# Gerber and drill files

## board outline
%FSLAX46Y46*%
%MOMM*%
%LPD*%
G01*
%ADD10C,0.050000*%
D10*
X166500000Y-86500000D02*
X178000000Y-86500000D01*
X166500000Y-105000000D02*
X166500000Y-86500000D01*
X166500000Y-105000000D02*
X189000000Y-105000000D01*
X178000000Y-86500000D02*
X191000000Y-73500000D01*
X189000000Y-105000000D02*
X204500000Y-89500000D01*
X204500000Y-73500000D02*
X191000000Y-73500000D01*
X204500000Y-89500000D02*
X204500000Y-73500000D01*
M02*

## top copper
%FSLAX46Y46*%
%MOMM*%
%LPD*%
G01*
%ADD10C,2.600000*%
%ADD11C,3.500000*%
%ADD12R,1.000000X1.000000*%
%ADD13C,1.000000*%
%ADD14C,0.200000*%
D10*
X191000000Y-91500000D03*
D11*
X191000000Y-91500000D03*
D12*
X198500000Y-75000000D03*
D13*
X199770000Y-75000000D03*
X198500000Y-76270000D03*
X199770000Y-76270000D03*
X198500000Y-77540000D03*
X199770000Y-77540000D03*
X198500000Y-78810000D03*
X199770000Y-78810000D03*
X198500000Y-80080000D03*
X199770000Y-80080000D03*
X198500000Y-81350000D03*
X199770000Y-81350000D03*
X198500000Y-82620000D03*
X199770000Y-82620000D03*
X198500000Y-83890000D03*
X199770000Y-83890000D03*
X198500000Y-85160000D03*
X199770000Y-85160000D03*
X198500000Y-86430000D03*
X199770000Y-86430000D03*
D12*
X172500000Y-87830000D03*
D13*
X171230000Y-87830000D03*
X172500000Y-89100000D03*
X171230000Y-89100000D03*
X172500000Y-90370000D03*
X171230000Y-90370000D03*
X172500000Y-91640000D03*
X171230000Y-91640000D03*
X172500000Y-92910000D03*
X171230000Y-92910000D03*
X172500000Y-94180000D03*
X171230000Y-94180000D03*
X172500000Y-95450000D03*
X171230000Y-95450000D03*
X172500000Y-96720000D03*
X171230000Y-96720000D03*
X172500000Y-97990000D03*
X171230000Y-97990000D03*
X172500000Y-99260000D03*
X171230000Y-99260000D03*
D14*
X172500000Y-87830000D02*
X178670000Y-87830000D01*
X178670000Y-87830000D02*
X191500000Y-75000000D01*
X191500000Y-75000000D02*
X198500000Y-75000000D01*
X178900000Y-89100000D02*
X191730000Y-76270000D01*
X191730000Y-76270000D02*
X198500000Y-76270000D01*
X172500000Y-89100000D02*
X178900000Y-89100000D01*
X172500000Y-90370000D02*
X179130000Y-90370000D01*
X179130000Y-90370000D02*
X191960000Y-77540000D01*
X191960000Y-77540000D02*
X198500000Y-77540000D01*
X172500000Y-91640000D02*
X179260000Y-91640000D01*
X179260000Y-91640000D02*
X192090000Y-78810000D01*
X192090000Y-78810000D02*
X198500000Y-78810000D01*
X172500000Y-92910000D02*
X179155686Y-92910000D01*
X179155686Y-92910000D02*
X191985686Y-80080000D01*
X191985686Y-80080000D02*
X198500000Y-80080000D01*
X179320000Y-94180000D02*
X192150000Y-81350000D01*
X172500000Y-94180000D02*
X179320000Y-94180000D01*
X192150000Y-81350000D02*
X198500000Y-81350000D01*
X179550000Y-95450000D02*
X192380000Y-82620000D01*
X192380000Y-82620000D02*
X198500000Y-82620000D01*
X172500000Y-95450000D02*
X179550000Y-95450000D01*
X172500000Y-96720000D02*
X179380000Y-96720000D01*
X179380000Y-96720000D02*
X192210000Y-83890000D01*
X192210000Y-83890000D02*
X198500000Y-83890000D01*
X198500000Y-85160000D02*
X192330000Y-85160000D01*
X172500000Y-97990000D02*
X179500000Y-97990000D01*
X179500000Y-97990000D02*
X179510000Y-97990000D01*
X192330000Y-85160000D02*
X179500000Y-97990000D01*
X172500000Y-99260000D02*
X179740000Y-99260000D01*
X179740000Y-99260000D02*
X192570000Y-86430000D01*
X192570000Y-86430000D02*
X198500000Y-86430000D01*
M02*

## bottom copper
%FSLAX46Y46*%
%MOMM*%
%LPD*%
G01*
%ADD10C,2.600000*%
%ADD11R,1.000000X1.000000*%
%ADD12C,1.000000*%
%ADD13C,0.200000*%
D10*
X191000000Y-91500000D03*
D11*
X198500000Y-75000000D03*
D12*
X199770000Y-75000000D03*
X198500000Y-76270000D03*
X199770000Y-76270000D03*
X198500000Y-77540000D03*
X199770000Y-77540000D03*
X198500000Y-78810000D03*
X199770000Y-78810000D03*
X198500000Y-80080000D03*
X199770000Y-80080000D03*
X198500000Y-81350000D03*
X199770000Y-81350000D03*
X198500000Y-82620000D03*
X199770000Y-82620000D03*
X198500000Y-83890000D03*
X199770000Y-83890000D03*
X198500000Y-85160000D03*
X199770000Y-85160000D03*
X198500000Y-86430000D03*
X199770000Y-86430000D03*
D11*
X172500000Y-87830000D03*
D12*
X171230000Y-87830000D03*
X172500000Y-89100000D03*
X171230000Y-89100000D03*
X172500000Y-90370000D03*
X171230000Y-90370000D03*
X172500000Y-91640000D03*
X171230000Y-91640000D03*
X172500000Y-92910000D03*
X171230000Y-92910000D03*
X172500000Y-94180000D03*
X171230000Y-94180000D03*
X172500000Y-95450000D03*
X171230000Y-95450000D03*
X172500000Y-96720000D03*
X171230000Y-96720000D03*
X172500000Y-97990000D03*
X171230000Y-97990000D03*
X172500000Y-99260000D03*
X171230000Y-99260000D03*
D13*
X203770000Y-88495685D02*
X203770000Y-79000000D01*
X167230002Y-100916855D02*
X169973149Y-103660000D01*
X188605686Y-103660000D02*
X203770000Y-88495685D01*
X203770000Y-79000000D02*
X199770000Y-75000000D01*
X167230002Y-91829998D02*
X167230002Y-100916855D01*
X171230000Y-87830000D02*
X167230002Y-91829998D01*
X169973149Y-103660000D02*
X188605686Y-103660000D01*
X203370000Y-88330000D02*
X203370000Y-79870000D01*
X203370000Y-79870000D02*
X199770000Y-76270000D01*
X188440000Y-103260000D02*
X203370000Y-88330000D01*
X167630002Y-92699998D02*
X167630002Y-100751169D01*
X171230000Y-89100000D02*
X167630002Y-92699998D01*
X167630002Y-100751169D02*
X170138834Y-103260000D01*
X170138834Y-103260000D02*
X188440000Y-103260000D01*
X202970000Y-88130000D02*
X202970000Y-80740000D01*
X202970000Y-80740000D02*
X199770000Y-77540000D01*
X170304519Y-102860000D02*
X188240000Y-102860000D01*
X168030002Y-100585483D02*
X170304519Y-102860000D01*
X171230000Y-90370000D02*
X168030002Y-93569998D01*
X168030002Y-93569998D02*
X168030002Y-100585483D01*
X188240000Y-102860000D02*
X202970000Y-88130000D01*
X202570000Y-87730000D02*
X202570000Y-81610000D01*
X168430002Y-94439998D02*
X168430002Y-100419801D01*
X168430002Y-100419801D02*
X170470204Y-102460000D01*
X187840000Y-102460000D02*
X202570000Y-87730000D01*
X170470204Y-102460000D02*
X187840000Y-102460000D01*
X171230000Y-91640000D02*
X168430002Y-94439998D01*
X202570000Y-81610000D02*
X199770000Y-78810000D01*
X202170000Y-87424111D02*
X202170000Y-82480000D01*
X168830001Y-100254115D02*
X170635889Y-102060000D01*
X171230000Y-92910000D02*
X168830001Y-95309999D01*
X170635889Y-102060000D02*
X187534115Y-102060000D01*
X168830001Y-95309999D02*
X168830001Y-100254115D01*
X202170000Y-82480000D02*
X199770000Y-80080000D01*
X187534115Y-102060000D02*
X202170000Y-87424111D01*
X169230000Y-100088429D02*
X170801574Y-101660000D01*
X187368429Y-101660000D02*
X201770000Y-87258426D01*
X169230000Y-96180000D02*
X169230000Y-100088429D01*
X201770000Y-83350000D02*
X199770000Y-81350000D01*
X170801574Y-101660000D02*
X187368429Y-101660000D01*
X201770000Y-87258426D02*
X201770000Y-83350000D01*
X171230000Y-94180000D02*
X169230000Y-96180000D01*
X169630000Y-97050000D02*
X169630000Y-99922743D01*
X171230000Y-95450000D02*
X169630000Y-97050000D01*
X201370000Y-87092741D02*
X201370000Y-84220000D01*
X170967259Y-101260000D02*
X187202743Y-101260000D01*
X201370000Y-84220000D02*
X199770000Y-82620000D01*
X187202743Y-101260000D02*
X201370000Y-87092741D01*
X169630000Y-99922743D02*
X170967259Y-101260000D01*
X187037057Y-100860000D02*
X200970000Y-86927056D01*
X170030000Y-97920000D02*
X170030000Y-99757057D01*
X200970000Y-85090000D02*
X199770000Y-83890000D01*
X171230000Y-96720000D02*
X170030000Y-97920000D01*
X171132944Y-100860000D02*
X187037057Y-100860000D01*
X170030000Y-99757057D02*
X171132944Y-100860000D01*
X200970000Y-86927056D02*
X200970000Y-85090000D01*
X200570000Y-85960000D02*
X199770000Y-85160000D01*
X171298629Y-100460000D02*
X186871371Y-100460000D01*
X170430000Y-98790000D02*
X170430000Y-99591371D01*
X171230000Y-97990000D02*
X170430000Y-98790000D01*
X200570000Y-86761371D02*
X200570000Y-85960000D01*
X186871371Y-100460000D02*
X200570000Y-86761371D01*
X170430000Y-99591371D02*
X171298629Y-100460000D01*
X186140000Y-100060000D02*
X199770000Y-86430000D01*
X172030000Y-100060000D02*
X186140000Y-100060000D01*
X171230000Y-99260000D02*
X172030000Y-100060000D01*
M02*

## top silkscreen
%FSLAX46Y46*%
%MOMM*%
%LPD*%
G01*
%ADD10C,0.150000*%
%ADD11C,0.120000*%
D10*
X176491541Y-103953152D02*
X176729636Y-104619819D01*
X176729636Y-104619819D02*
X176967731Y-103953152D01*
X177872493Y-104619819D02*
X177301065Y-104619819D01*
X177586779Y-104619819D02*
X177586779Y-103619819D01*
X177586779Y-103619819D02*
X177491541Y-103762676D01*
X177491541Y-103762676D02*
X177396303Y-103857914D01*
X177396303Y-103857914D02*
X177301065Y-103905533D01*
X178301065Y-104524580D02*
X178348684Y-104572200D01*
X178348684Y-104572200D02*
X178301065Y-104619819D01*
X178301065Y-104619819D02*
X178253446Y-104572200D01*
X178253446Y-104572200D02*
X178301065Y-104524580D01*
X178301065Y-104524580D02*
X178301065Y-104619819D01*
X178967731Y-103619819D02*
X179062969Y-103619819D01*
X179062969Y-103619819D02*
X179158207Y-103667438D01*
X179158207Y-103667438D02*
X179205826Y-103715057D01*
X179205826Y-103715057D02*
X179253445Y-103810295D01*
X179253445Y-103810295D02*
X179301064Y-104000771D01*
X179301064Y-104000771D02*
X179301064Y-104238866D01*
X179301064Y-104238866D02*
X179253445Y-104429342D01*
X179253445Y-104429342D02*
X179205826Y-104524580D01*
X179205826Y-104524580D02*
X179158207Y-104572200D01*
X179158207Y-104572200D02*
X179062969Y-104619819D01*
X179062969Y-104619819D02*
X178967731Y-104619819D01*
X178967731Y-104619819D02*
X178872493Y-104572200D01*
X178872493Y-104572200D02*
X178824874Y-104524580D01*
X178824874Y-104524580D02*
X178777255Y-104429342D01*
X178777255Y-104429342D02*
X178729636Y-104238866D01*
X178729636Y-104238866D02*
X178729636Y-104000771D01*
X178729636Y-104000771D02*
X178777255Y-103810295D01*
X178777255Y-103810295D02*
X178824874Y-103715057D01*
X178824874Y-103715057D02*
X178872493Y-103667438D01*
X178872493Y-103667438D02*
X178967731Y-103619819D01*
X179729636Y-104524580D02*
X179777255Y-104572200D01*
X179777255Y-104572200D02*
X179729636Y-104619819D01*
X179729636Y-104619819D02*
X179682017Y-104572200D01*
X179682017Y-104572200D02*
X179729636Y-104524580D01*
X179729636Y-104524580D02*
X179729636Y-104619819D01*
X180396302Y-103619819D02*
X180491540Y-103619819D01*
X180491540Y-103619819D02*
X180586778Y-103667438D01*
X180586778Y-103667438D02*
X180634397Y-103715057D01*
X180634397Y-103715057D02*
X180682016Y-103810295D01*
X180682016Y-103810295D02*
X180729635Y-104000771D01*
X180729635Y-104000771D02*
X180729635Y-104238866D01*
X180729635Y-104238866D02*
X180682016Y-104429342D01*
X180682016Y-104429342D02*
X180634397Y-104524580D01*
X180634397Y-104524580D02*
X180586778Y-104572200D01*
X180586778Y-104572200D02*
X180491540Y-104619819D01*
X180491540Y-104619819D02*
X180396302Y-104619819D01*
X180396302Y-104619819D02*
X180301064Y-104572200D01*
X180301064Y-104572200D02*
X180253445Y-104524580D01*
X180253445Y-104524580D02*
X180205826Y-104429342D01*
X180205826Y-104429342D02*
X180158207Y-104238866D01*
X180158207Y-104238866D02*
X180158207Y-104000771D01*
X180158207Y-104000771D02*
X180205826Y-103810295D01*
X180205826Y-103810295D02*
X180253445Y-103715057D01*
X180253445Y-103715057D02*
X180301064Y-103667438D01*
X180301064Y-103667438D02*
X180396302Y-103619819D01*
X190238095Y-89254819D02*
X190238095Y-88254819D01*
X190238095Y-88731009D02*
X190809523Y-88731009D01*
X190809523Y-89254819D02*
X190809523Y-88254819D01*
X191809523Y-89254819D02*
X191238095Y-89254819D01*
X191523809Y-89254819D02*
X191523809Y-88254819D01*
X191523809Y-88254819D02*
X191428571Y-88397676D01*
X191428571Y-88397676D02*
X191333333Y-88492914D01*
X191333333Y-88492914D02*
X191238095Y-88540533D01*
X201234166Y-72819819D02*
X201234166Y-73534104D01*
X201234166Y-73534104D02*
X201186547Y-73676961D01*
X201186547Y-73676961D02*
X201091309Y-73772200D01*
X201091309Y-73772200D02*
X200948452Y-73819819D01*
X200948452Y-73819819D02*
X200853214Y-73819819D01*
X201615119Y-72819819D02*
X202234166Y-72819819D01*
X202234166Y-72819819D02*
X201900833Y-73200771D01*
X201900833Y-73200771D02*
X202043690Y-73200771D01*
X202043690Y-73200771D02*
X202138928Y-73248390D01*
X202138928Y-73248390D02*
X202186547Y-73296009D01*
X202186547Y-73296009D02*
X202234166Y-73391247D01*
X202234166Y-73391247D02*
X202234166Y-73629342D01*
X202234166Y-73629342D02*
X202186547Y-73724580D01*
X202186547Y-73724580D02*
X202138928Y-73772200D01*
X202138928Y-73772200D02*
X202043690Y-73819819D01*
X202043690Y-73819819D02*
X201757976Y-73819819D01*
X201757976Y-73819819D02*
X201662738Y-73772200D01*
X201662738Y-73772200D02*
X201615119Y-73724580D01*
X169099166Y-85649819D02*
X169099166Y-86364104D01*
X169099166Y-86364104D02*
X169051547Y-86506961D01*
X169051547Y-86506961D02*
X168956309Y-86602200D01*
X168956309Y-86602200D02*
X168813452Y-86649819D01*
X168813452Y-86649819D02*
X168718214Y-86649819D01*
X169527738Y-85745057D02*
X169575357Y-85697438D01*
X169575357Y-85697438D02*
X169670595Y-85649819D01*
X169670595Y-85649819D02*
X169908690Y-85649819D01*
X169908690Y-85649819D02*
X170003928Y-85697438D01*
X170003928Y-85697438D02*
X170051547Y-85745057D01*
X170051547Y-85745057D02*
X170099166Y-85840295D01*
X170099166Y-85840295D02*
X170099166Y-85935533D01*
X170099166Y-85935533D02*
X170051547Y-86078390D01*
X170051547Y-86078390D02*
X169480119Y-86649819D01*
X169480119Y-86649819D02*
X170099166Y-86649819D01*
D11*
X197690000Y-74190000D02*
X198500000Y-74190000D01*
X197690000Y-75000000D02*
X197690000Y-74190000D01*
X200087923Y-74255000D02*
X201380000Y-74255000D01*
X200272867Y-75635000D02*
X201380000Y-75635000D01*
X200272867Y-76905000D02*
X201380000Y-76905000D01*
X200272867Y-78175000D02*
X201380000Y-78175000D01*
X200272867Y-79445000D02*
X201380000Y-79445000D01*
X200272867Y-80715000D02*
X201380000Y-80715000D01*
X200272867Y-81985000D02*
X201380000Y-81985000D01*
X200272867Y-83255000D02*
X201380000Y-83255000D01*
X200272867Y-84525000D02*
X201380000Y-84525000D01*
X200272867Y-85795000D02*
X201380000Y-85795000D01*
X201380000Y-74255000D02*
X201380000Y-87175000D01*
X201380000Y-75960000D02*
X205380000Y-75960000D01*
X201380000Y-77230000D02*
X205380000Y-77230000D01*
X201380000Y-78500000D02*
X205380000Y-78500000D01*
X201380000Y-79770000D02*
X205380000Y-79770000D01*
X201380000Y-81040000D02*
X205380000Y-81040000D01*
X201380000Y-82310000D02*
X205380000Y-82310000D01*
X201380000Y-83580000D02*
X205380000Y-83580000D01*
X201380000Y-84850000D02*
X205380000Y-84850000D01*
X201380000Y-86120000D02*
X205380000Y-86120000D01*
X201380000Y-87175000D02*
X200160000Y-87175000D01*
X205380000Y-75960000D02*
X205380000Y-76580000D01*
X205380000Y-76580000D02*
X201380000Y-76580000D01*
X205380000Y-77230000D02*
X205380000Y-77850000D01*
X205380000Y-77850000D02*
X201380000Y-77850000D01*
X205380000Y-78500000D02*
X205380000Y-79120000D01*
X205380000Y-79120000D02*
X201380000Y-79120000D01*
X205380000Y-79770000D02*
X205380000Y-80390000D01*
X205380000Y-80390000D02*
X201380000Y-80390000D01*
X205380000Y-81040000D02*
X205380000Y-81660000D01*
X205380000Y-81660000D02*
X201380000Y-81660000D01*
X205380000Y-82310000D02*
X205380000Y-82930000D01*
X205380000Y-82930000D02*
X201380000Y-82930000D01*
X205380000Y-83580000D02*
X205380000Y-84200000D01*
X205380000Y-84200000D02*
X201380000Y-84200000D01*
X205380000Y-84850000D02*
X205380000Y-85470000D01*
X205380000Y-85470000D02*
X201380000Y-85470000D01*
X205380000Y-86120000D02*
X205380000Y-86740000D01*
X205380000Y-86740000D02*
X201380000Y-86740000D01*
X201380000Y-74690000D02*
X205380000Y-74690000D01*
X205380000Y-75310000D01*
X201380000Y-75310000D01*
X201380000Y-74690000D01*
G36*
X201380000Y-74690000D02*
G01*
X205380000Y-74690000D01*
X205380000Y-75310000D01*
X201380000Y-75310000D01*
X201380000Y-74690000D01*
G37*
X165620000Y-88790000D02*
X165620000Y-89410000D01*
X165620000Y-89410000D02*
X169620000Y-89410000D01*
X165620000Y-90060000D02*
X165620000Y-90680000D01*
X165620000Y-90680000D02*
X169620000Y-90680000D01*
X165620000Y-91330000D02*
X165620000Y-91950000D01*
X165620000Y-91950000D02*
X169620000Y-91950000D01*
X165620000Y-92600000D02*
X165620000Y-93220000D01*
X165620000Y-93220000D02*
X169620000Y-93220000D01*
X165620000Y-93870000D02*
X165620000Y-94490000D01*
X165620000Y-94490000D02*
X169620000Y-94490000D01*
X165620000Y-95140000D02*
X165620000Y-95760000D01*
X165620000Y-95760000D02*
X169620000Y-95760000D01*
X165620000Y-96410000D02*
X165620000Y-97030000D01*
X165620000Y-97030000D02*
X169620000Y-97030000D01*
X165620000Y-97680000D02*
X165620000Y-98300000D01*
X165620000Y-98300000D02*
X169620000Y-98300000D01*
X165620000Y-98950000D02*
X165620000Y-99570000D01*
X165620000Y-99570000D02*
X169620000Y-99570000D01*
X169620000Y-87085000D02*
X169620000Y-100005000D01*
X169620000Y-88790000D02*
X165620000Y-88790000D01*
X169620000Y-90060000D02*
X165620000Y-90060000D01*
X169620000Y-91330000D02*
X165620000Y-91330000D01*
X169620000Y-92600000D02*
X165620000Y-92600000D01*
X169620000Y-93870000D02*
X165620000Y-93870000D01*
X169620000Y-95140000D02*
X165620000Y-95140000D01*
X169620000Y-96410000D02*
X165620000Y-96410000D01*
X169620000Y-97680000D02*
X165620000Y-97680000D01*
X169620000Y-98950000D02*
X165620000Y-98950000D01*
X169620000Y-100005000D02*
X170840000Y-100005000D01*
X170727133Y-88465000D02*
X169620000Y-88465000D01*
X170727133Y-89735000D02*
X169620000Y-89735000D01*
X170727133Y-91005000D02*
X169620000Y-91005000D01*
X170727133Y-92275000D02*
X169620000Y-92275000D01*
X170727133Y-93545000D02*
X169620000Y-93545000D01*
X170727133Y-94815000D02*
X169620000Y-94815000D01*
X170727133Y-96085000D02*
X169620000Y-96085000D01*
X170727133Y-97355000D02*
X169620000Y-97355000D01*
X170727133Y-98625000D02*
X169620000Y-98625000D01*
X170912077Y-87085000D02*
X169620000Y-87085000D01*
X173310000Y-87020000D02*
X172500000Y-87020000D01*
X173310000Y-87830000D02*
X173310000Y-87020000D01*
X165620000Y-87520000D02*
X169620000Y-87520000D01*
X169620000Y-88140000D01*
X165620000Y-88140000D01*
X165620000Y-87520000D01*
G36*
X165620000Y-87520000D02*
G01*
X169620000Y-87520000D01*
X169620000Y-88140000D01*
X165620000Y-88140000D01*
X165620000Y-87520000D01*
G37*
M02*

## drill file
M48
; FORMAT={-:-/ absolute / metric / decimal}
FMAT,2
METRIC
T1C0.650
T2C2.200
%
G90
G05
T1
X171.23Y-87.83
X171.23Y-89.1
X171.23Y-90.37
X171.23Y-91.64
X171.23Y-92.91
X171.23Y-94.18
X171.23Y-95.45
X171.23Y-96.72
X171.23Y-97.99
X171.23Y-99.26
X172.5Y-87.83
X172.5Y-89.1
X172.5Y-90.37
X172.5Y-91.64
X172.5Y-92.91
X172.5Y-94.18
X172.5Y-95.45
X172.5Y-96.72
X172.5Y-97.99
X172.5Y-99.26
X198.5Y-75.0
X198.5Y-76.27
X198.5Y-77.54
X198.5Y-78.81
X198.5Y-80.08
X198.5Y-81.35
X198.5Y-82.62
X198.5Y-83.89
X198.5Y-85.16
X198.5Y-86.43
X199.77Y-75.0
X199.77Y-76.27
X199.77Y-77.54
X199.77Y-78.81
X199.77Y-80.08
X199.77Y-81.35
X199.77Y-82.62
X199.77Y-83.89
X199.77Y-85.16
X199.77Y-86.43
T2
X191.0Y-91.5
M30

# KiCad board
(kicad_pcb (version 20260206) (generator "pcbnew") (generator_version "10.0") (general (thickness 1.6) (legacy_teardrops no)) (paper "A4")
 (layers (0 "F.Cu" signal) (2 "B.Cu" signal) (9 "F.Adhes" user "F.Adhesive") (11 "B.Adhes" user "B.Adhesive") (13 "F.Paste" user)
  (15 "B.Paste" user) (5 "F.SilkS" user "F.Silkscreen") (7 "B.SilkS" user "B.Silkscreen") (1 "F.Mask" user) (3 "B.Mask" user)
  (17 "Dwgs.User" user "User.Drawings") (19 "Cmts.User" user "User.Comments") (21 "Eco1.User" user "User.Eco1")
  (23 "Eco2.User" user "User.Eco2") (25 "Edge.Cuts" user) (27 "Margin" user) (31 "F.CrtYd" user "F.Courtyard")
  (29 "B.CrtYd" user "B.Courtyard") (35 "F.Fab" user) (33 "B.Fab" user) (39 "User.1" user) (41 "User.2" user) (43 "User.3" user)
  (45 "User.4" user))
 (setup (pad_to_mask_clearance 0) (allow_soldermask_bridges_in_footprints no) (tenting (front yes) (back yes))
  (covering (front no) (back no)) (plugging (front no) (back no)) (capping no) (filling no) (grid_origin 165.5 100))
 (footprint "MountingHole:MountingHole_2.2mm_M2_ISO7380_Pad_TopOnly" (layer "F.Cu") (at 191 91.5)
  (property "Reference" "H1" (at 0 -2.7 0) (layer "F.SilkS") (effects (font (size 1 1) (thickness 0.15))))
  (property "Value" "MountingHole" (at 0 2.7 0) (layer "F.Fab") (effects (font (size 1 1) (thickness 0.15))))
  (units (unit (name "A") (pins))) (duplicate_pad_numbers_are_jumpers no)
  (pad "1" thru_hole circle (at 0 0) (size 2.6 2.6) (drill 2.2) (layers "*.Cu" "*.Mask") (remove_unused_layers no) (zone_connect 2))
  (pad "1" connect circle (at 0 0) (size 3.5 3.5) (layers "F.Cu" "F.Mask") (zone_connect 2)))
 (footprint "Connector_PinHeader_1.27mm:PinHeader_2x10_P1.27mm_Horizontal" (layer "F.Cu") (at 198.5 75)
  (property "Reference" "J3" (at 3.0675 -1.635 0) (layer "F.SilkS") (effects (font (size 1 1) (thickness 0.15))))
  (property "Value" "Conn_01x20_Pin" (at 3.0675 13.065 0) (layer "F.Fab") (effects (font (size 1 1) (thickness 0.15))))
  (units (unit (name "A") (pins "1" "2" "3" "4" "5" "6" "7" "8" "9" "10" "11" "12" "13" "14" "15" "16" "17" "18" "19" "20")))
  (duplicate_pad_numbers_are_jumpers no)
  (fp_line (start -0.81 -0.81) (end 0 -0.81) (stroke (width 0.12) (type solid)) (layer "F.SilkS"))
  (fp_line (start -0.81 0) (end -0.81 -0.81) (stroke (width 0.12) (type solid)) (layer "F.SilkS"))
  (fp_line (start 1.587923 -0.745) (end 2.88 -0.745) (stroke (width 0.12) (type solid)) (layer "F.SilkS"))
  (fp_line (start 1.772867 0.635) (end 2.88 0.635) (stroke (width 0.12) (type solid)) (layer "F.SilkS"))
  (fp_line (start 1.772867 1.905) (end 2.88 1.905) (stroke (width 0.12) (type solid)) (layer "F.SilkS"))
  (fp_line (start 1.772867 3.175) (end 2.88 3.175) (stroke (width 0.12) (type solid)) (layer "F.SilkS"))
  (fp_line (start 1.772867 4.445) (end 2.88 4.445) (stroke (width 0.12) (type solid)) (layer "F.SilkS"))
  (fp_line (start 1.772867 5.715) (end 2.88 5.715) (stroke (width 0.12) (type solid)) (layer "F.SilkS"))
  (fp_line (start 1.772867 6.985) (end 2.88 6.985) (stroke (width 0.12) (type solid)) (layer "F.SilkS"))
  (fp_line (start 1.772867 8.255) (end 2.88 8.255) (stroke (width 0.12) (type solid)) (layer "F.SilkS"))
  (fp_line (start 1.772867 9.525) (end 2.88 9.525) (stroke (width 0.12) (type solid)) (layer "F.SilkS"))
  (fp_line (start 1.772867 10.795) (end 2.88 10.795) (stroke (width 0.12) (type solid)) (layer "F.SilkS"))
  (fp_line (start 2.88 -0.745) (end 2.88 12.175) (stroke (width 0.12) (type solid)) (layer "F.SilkS"))
  (fp_line (start 2.88 0.96) (end 6.88 0.96) (stroke (width 0.12) (type solid)) (layer "F.SilkS"))
  (fp_line (start 2.88 2.23) (end 6.88 2.23) (stroke (width 0.12) (type solid)) (layer "F.SilkS"))
  (fp_line (start 2.88 3.5) (end 6.88 3.5) (stroke (width 0.12) (type solid)) (layer "F.SilkS"))
  (fp_line (start 2.88 4.77) (end 6.88 4.77) (stroke (width 0.12) (type solid)) (layer "F.SilkS"))
  (fp_line (start 2.88 6.04) (end 6.88 6.04) (stroke (width 0.12) (type solid)) (layer "F.SilkS"))
  (fp_line (start 2.88 7.31) (end 6.88 7.31) (stroke (width 0.12) (type solid)) (layer "F.SilkS"))
  (fp_line (start 2.88 8.58) (end 6.88 8.58) (stroke (width 0.12) (type solid)) (layer "F.SilkS"))
  (fp_line (start 2.88 9.85) (end 6.88 9.85) (stroke (width 0.12) (type solid)) (layer "F.SilkS"))
  (fp_line (start 2.88 11.12) (end 6.88 11.12) (stroke (width 0.12) (type solid)) (layer "F.SilkS"))
  (fp_line (start 2.88 12.175) (end 1.66 12.175) (stroke (width 0.12) (type solid)) (layer "F.SilkS"))
  (fp_line (start 6.88 0.96) (end 6.88 1.58) (stroke (width 0.12) (type solid)) (layer "F.SilkS"))
  (fp_line (start 6.88 1.58) (end 2.88 1.58) (stroke (width 0.12) (type solid)) (layer "F.SilkS"))
  (fp_line (start 6.88 2.23) (end 6.88 2.85) (stroke (width 0.12) (type solid)) (layer "F.SilkS"))
  (fp_line (start 6.88 2.85) (end 2.88 2.85) (stroke (width 0.12) (type solid)) (layer "F.SilkS"))
  (fp_line (start 6.88 3.5) (end 6.88 4.12) (stroke (width 0.12) (type solid)) (layer "F.SilkS"))
  (fp_line (start 6.88 4.12) (end 2.88 4.12) (stroke (width 0.12) (type solid)) (layer "F.SilkS"))
  (fp_line (start 6.88 4.77) (end 6.88 5.39) (stroke (width 0.12) (type solid)) (layer "F.SilkS"))
  (fp_line (start 6.88 5.39) (end 2.88 5.39) (stroke (width 0.12) (type solid)) (layer "F.SilkS"))
  (fp_line (start 6.88 6.04) (end 6.88 6.66) (stroke (width 0.12) (type solid)) (layer "F.SilkS"))
  (fp_line (start 6.88 6.66) (end 2.88 6.66) (stroke (width 0.12) (type solid)) (layer "F.SilkS"))
  (fp_line (start 6.88 7.31) (end 6.88 7.93) (stroke (width 0.12) (type solid)) (layer "F.SilkS"))
  (fp_line (start 6.88 7.93) (end 2.88 7.93) (stroke (width 0.12) (type solid)) (layer "F.SilkS"))
  (fp_line (start 6.88 8.58) (end 6.88 9.2) (stroke (width 0.12) (type solid)) (layer "F.SilkS"))
  (fp_line (start 6.88 9.2) (end 2.88 9.2) (stroke (width 0.12) (type solid)) (layer "F.SilkS"))
  (fp_line (start 6.88 9.85) (end 6.88 10.47) (stroke (width 0.12) (type solid)) (layer "F.SilkS"))
  (fp_line (start 6.88 10.47) (end 2.88 10.47) (stroke (width 0.12) (type solid)) (layer "F.SilkS"))
  (fp_line (start 6.88 11.12) (end 6.88 11.74) (stroke (width 0.12) (type solid)) (layer "F.SilkS"))
  (fp_line (start 6.88 11.74) (end 2.88 11.74) (stroke (width 0.12) (type solid)) (layer "F.SilkS"))
  (fp_rect (start 2.88 -0.31) (end 6.88 0.31) (stroke (width 0.12) (type solid)) (fill yes) (layer "F.SilkS"))
  (pad "1" thru_hole rect (at 0 0) (size 1 1) (drill 0.65) (layers "*.Cu" "*.Mask") (remove_unused_layers no) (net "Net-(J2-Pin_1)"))
  (pad "2" thru_hole circle (at 1.27 0) (size 1 1) (drill 0.65) (layers "*.Cu" "*.Mask") (remove_unused_layers no) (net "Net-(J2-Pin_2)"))
  (pad "3" thru_hole circle (at 0 1.27) (size 1 1) (drill 0.65) (layers "*.Cu" "*.Mask") (remove_unused_layers no) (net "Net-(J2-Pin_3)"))
  (pad "4" thru_hole circle (at 1.27 1.27) (size 1 1) (drill 0.65) (layers "*.Cu" "*.Mask") (remove_unused_layers no) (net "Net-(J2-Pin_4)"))
  (pad "5" thru_hole circle (at 0 2.54) (size 1 1) (drill 0.65) (layers "*.Cu" "*.Mask") (remove_unused_layers no) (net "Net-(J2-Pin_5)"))
  (pad "6" thru_hole circle (at 1.27 2.54) (size 1 1) (drill 0.65) (layers "*.Cu" "*.Mask") (remove_unused_layers no) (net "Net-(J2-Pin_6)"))
  (pad "7" thru_hole circle (at 0 3.81) (size 1 1) (drill 0.65) (layers "*.Cu" "*.Mask") (remove_unused_layers no) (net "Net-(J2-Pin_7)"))
  (pad "8" thru_hole circle (at 1.27 3.81) (size 1 1) (drill 0.65) (layers "*.Cu" "*.Mask") (remove_unused_layers no) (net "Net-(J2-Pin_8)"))
  (pad "9" thru_hole circle (at 0 5.08) (size 1 1) (drill 0.65) (layers "*.Cu" "*.Mask") (remove_unused_layers no) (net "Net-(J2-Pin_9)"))
  (pad "10" thru_hole circle (at 1.27 5.08) (size 1 1) (drill 0.65) (layers "*.Cu" "*.Mask") (remove_unused_layers no)
   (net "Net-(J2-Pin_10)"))
  (pad "11" thru_hole circle (at 0 6.35) (size 1 1) (drill 0.65) (layers "*.Cu" "*.Mask") (remove_unused_layers no) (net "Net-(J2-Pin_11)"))
  (pad "12" thru_hole circle (at 1.27 6.35) (size 1 1) (drill 0.65) (layers "*.Cu" "*.Mask") (remove_unused_layers no)
   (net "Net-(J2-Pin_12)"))
  (pad "13" thru_hole circle (at 0 7.62) (size 1 1) (drill 0.65) (layers "*.Cu" "*.Mask") (remove_unused_layers no) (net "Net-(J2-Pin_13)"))
  (pad "14" thru_hole circle (at 1.27 7.62) (size 1 1) (drill 0.65) (layers "*.Cu" "*.Mask") (remove_unused_layers no)
   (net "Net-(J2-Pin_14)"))
  (pad "15" thru_hole circle (at 0 8.89) (size 1 1) (drill 0.65) (layers "*.Cu" "*.Mask") (remove_unused_layers no) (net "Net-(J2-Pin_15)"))
  (pad "16" thru_hole circle (at 1.27 8.89) (size 1 1) (drill 0.65) (layers "*.Cu" "*.Mask") (remove_unused_layers no)
   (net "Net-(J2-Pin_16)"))
  (pad "17" thru_hole circle (at 0 10.16) (size 1 1) (drill 0.65) (layers "*.Cu" "*.Mask") (remove_unused_layers no) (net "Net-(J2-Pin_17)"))
  (pad "18" thru_hole circle (at 1.27 10.16) (size 1 1) (drill 0.65) (layers "*.Cu" "*.Mask") (remove_unused_layers no)
   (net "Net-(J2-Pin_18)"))
  (pad "19" thru_hole circle (at 0 11.43) (size 1 1) (drill 0.65) (layers "*.Cu" "*.Mask") (remove_unused_layers no) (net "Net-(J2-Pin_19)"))
  (pad "20" thru_hole circle (at 1.27 11.43) (size 1 1) (drill 0.65) (layers "*.Cu" "*.Mask") (remove_unused_layers no)
   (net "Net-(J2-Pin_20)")))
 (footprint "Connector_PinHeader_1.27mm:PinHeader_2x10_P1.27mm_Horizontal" (layer "F.Cu") (at 172.5 87.83)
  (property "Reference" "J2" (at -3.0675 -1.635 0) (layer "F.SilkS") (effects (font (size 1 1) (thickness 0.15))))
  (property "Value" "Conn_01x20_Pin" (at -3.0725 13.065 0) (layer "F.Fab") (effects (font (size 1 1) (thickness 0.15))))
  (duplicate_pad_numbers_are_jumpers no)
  (fp_line (start -6.88 0.96) (end -6.88 1.58) (stroke (width 0.12) (type solid)) (layer "F.SilkS"))
  (fp_line (start -6.88 1.58) (end -2.88 1.58) (stroke (width 0.12) (type solid)) (layer "F.SilkS"))
  (fp_line (start -6.88 2.23) (end -6.88 2.85) (stroke (width 0.12) (type solid)) (layer "F.SilkS"))
  (fp_line (start -6.88 2.85) (end -2.88 2.85) (stroke (width 0.12) (type solid)) (layer "F.SilkS"))
  (fp_line (start -6.88 3.5) (end -6.88 4.12) (stroke (width 0.12) (type solid)) (layer "F.SilkS"))
  (fp_line (start -6.88 4.12) (end -2.88 4.12) (stroke (width 0.12) (type solid)) (layer "F.SilkS"))
  (fp_line (start -6.88 4.77) (end -6.88 5.39) (stroke (width 0.12) (type solid)) (layer "F.SilkS"))
  (fp_line (start -6.88 5.39) (end -2.88 5.39) (stroke (width 0.12) (type solid)) (layer "F.SilkS"))
  (fp_line (start -6.88 6.04) (end -6.88 6.66) (stroke (width 0.12) (type solid)) (layer "F.SilkS"))
  (fp_line (start -6.88 6.66) (end -2.88 6.66) (stroke (width 0.12) (type solid)) (layer "F.SilkS"))
  (fp_line (start -6.88 7.31) (end -6.88 7.93) (stroke (width 0.12) (type solid)) (layer "F.SilkS"))
  (fp_line (start -6.88 7.93) (end -2.88 7.93) (stroke (width 0.12) (type solid)) (layer "F.SilkS"))
  (fp_line (start -6.88 8.58) (end -6.88 9.2) (stroke (width 0.12) (type solid)) (layer "F.SilkS"))
  (fp_line (start -6.88 9.2) (end -2.88 9.2) (stroke (width 0.12) (type solid)) (layer "F.SilkS"))
  (fp_line (start -6.88 9.85) (end -6.88 10.47) (stroke (width 0.12) (type solid)) (layer "F.SilkS"))
  (fp_line (start -6.88 10.47) (end -2.88 10.47) (stroke (width 0.12) (type solid)) (layer "F.SilkS"))
  (fp_line (start -6.88 11.12) (end -6.88 11.74) (stroke (width 0.12) (type solid)) (layer "F.SilkS"))
  (fp_line (start -6.88 11.74) (end -2.88 11.74) (stroke (width 0.12) (type solid)) (layer "F.SilkS"))
  (fp_line (start -2.88 -0.745) (end -2.88 12.175) (stroke (width 0.12) (type solid)) (layer "F.SilkS"))
  (fp_line (start -2.88 0.96) (end -6.88 0.96) (stroke (width 0.12) (type solid)) (layer "F.SilkS"))
  (fp_line (start -2.88 2.23) (end -6.88 2.23) (stroke (width 0.12) (type solid)) (layer "F.SilkS"))
  (fp_line (start -2.88 3.5) (end -6.88 3.5) (stroke (width 0.12) (type solid)) (layer "F.SilkS"))
  (fp_line (start -2.88 4.77) (end -6.88 4.77) (stroke (width 0.12) (type solid)) (layer "F.SilkS"))
  (fp_line (start -2.88 6.04) (end -6.88 6.04) (stroke (width 0.12) (type solid)) (layer "F.SilkS"))
  (fp_line (start -2.88 7.31) (end -6.88 7.31) (stroke (width 0.12) (type solid)) (layer "F.SilkS"))
  (fp_line (start -2.88 8.58) (end -6.88 8.58) (stroke (width 0.12) (type solid)) (layer "F.SilkS"))
  (fp_line (start -2.88 9.85) (end -6.88 9.85) (stroke (width 0.12) (type solid)) (layer "F.SilkS"))
  (fp_line (start -2.88 11.12) (end -6.88 11.12) (stroke (width 0.12) (type solid)) (layer "F.SilkS"))
  (fp_line (start -2.88 12.175) (end -1.66 12.175) (stroke (width 0.12) (type solid)) (layer "F.SilkS"))
  (fp_line (start -1.772867 0.635) (end -2.88 0.635) (stroke (width 0.12) (type solid)) (layer "F.SilkS"))
  (fp_line (start -1.772867 1.905) (end -2.88 1.905) (stroke (width 0.12) (type solid)) (layer "F.SilkS"))
  (fp_line (start -1.772867 3.175) (end -2.88 3.175) (stroke (width 0.12) (type solid)) (layer "F.SilkS"))
  (fp_line (start -1.772867 4.445) (end -2.88 4.445) (stroke (width 0.12) (type solid)) (layer "F.SilkS"))
  (fp_line (start -1.772867 5.715) (end -2.88 5.715) (stroke (width 0.12) (type solid)) (layer "F.SilkS"))
  (fp_line (start -1.772867 6.985) (end -2.88 6.985) (stroke (width 0.12) (type solid)) (layer "F.SilkS"))
  (fp_line (start -1.772867 8.255) (end -2.88 8.255) (stroke (width 0.12) (type solid)) (layer "F.SilkS"))
  (fp_line (start -1.772867 9.525) (end -2.88 9.525) (stroke (width 0.12) (type solid)) (layer "F.SilkS"))
  (fp_line (start -1.772867 10.795) (end -2.88 10.795) (stroke (width 0.12) (type solid)) (layer "F.SilkS"))
  (fp_line (start -1.587923 -0.745) (end -2.88 -0.745) (stroke (width 0.12) (type solid)) (layer "F.SilkS"))
  (fp_line (start 0.81 -0.81) (end 0 -0.81) (stroke (width 0.12) (type solid)) (layer "F.SilkS"))
  (fp_line (start 0.81 0) (end 0.81 -0.81) (stroke (width 0.12) (type solid)) (layer "F.SilkS"))
  (fp_rect (start -2.88 -0.31) (end -6.88 0.31) (stroke (width 0.12) (type solid)) (fill yes) (layer "F.SilkS"))
  (pad "1" thru_hole rect (at 0 0) (size 1 1) (drill 0.65) (layers "*.Cu" "*.Mask") (remove_unused_layers no) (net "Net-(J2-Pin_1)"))
  (pad "2" thru_hole circle (at -1.27 0) (size 1 1) (drill 0.65) (layers "*.Cu" "*.Mask") (remove_unused_layers no) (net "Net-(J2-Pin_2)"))
  (pad "3" thru_hole circle (at 0 1.27) (size 1 1) (drill 0.65) (layers "*.Cu" "*.Mask") (remove_unused_layers no) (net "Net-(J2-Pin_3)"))
  (pad "4" thru_hole circle (at -1.27 1.27) (size 1 1) (drill 0.65) (layers "*.Cu" "*.Mask") (remove_unused_layers no)
   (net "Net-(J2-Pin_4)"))
  (pad "5" thru_hole circle (at 0 2.54) (size 1 1) (drill 0.65) (layers "*.Cu" "*.Mask") (remove_unused_layers no) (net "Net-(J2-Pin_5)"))
  (pad "6" thru_hole circle (at -1.27 2.54) (size 1 1) (drill 0.65) (layers "*.Cu" "*.Mask") (remove_unused_layers no)
   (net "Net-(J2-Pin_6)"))
  (pad "7" thru_hole circle (at 0 3.81) (size 1 1) (drill 0.65) (layers "*.Cu" "*.Mask") (remove_unused_layers no) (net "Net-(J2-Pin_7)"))
  (pad "8" thru_hole circle (at -1.27 3.81) (size 1 1) (drill 0.65) (layers "*.Cu" "*.Mask") (remove_unused_layers no)
   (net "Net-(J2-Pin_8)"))
  (pad "9" thru_hole circle (at 0 5.08) (size 1 1) (drill 0.65) (layers "*.Cu" "*.Mask") (remove_unused_layers no) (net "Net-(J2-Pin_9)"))
  (pad "10" thru_hole circle (at -1.27 5.08) (size 1 1) (drill 0.65) (layers "*.Cu" "*.Mask") (remove_unused_layers no)
   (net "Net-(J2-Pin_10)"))
  (pad "11" thru_hole circle (at 0 6.35) (size 1 1) (drill 0.65) (layers "*.Cu" "*.Mask") (remove_unused_layers no) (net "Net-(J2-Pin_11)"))
  (pad "12" thru_hole circle (at -1.27 6.35) (size 1 1) (drill 0.65) (layers "*.Cu" "*.Mask") (remove_unused_layers no)
   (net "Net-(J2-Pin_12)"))
  (pad "13" thru_hole circle (at 0 7.62) (size 1 1) (drill 0.65) (layers "*.Cu" "*.Mask") (remove_unused_layers no) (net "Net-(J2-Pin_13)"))
  (pad "14" thru_hole circle (at -1.27 7.62) (size 1 1) (drill 0.65) (layers "*.Cu" "*.Mask") (remove_unused_layers no)
   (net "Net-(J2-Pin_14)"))
  (pad "15" thru_hole circle (at 0 8.89) (size 1 1) (drill 0.65) (layers "*.Cu" "*.Mask") (remove_unused_layers no) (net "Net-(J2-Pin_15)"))
  (pad "16" thru_hole circle (at -1.27 8.89) (size 1 1) (drill 0.65) (layers "*.Cu" "*.Mask") (remove_unused_layers no)
   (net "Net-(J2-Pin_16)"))
  (pad "17" thru_hole circle (at 0 10.16) (size 1 1) (drill 0.65) (layers "*.Cu" "*.Mask") (remove_unused_layers no) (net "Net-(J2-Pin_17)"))
  (pad "18" thru_hole circle (at -1.27 10.16) (size 1 1) (drill 0.65) (layers "*.Cu" "*.Mask") (remove_unused_layers no)
   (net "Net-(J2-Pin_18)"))
  (pad "19" thru_hole circle (at 0 11.43) (size 1 1) (drill 0.65) (layers "*.Cu" "*.Mask") (remove_unused_layers no) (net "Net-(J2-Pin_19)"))
  (pad "20" thru_hole circle (at -1.27 11.43) (size 1 1) (drill 0.65) (layers "*.Cu" "*.Mask") (remove_unused_layers no)
   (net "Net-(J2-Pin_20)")))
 (gr_line (start 166.5 86.5) (end 178 86.5) (stroke (width 0.05) (type default)) (layer "Edge.Cuts"))
 (gr_line (start 166.5 105) (end 166.5 86.5) (stroke (width 0.05) (type default)) (layer "Edge.Cuts"))
 (gr_line (start 166.5 105) (end 189 105) (stroke (width 0.05) (type default)) (layer "Edge.Cuts"))
 (gr_line (start 178 86.5) (end 191 73.5) (stroke (width 0.05) (type default)) (layer "Edge.Cuts"))
 (gr_line (start 189 105) (end 204.5 89.5) (stroke (width 0.05) (type default)) (layer "Edge.Cuts"))
 (gr_line (start 204.5 73.5) (end 191 73.5) (stroke (width 0.05) (type default)) (layer "Edge.Cuts"))
 (gr_line (start 204.5 89.5) (end 204.5 73.5) (stroke (width 0.05) (type default)) (layer "Edge.Cuts"))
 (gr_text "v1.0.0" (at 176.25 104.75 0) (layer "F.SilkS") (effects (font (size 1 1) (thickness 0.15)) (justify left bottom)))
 (segment (start 172.5 87.83) (end 178.67 87.83) (width 0.2) (layer "F.Cu") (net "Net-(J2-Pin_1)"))
 (segment (start 178.67 87.83) (end 191.5 75) (width 0.2) (layer "F.Cu") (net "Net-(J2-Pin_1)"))
 (segment (start 191.5 75) (end 198.5 75) (width 0.2) (layer "F.Cu") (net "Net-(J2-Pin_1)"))
 (segment (start 203.77 88.495685) (end 203.77 79) (width 0.2) (layer "B.Cu") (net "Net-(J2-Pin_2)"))
 (segment (start 167.230002 100.916855) (end 169.973149 103.66) (width 0.2) (layer "B.Cu") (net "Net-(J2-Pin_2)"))
 (segment (start 188.605686 103.66) (end 203.77 88.495685) (width 0.2) (layer "B.Cu") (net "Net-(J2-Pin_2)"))
 (segment (start 203.77 79) (end 199.77 75) (width 0.2) (layer "B.Cu") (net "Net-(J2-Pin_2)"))
 (segment (start 167.230002 91.829998) (end 167.230002 100.916855) (width 0.2) (layer "B.Cu") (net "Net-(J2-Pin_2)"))
 (segment (start 171.23 87.83) (end 167.230002 91.829998) (width 0.2) (layer "B.Cu") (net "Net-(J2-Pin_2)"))
 (segment (start 169.973149 103.66) (end 188.605686 103.66) (width 0.2) (layer "B.Cu") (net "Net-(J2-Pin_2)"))
 (segment (start 178.9 89.1) (end 191.73 76.27) (width 0.2) (layer "F.Cu") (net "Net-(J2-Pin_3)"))
 (segment (start 191.73 76.27) (end 198.5 76.27) (width 0.2) (layer "F.Cu") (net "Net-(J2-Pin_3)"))
 (segment (start 172.5 89.1) (end 178.9 89.1) (width 0.2) (layer "F.Cu") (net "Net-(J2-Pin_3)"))
 (segment (start 203.37 88.33) (end 203.37 79.87) (width 0.2) (layer "B.Cu") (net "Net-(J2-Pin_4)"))
 (segment (start 203.37 79.87) (end 199.77 76.27) (width 0.2) (layer "B.Cu") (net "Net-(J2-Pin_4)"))
 (segment (start 188.44 103.26) (end 203.37 88.33) (width 0.2) (layer "B.Cu") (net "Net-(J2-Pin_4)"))
 (segment (start 167.630002 92.699998) (end 167.630002 100.751169) (width 0.2) (layer "B.Cu") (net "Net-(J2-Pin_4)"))
 (segment (start 171.23 89.1) (end 167.630002 92.699998) (width 0.2) (layer "B.Cu") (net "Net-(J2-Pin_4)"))
 (segment (start 167.630002 100.751169) (end 170.138834 103.26) (width 0.2) (layer "B.Cu") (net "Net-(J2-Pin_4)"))
 (segment (start 170.138834 103.26) (end 188.44 103.26) (width 0.2) (layer "B.Cu") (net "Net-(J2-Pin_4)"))
 (segment (start 172.5 90.37) (end 179.13 90.37) (width 0.2) (layer "F.Cu") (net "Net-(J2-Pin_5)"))
 (segment (start 179.13 90.37) (end 191.96 77.54) (width 0.2) (layer "F.Cu") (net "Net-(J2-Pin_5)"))
 (segment (start 191.96 77.54) (end 198.5 77.54) (width 0.2) (layer "F.Cu") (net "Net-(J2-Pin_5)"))
 (segment (start 202.97 88.13) (end 202.97 80.74) (width 0.2) (layer "B.Cu") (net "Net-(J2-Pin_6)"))
 (segment (start 202.97 80.74) (end 199.77 77.54) (width 0.2) (layer "B.Cu") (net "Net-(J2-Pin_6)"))
 (segment (start 170.304519 102.86) (end 188.24 102.86) (width 0.2) (layer "B.Cu") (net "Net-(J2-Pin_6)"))
 (segment (start 168.030002 100.585483) (end 170.304519 102.86) (width 0.2) (layer "B.Cu") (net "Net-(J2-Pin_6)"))
 (segment (start 171.23 90.37) (end 168.030002 93.569998) (width 0.2) (layer "B.Cu") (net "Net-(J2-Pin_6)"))
 (segment (start 168.030002 93.569998) (end 168.030002 100.585483) (width 0.2) (layer "B.Cu") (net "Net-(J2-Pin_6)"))
 (segment (start 188.24 102.86) (end 202.97 88.13) (width 0.2) (layer "B.Cu") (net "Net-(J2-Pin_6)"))
 (segment (start 172.5 91.64) (end 179.26 91.64) (width 0.2) (layer "F.Cu") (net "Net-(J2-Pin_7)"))
 (segment (start 179.26 91.64) (end 192.09 78.81) (width 0.2) (layer "F.Cu") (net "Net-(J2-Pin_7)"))
 (segment (start 192.09 78.81) (end 198.5 78.81) (width 0.2) (layer "F.Cu") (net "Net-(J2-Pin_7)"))
 (segment (start 202.57 87.73) (end 202.57 81.61) (width 0.2) (layer "B.Cu") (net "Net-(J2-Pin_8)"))
 (segment (start 168.430002 94.439998) (end 168.430002 100.419801) (width 0.2) (layer "B.Cu") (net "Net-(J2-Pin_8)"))
 (segment (start 168.430002 100.419801) (end 170.470204 102.46) (width 0.2) (layer "B.Cu") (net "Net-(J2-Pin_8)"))
 (segment (start 187.84 102.46) (end 202.57 87.73) (width 0.2) (layer "B.Cu") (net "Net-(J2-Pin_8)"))
 (segment (start 170.470204 102.46) (end 187.84 102.46) (width 0.2) (layer "B.Cu") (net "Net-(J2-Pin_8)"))
 (segment (start 171.23 91.64) (end 168.430002 94.439998) (width 0.2) (layer "B.Cu") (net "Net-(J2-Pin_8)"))
 (segment (start 202.57 81.61) (end 199.77 78.81) (width 0.2) (layer "B.Cu") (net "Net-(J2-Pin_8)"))
 (segment (start 172.5 92.91) (end 179.155686 92.91) (width 0.2) (layer "F.Cu") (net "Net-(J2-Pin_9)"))
 (segment (start 179.155686 92.91) (end 191.985686 80.08) (width 0.2) (layer "F.Cu") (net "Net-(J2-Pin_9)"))
 (segment (start 191.985686 80.08) (end 198.5 80.08) (width 0.2) (layer "F.Cu") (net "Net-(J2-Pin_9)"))
 (segment (start 202.17 87.424111) (end 202.17 82.48) (width 0.2) (layer "B.Cu") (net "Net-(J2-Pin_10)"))
 (segment (start 168.830001 100.254115) (end 170.635889 102.06) (width 0.2) (layer "B.Cu") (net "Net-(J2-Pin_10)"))
 (segment (start 171.23 92.91) (end 168.830001 95.309999) (width 0.2) (layer "B.Cu") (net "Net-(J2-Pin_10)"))
 (segment (start 170.635889 102.06) (end 187.534115 102.06) (width 0.2) (layer "B.Cu") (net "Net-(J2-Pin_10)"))
 (segment (start 168.830001 95.309999) (end 168.830001 100.254115) (width 0.2) (layer "B.Cu") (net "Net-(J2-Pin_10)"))
 (segment (start 202.17 82.48) (end 199.77 80.08) (width 0.2) (layer "B.Cu") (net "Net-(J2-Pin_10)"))
 (segment (start 187.534115 102.06) (end 202.17 87.424111) (width 0.2) (layer "B.Cu") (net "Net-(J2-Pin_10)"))
 (segment (start 179.32 94.18) (end 192.15 81.35) (width 0.2) (layer "F.Cu") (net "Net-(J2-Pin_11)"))
 (segment (start 172.5 94.18) (end 179.32 94.18) (width 0.2) (layer "F.Cu") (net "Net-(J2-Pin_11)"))
 (segment (start 192.15 81.35) (end 198.5 81.35) (width 0.2) (layer "F.Cu") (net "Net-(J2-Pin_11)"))
 (segment (start 169.23 100.088429) (end 170.801574 101.66) (width 0.2) (layer "B.Cu") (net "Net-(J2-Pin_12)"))
 (segment (start 187.368429 101.66) (end 201.77 87.258426) (width 0.2) (layer "B.Cu") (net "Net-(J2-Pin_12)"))
 (segment (start 169.23 96.18) (end 169.23 100.088429) (width 0.2) (layer "B.Cu") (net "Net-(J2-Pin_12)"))
 (segment (start 201.77 83.35) (end 199.77 81.35) (width 0.2) (layer "B.Cu") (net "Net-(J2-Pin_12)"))
 (segment (start 170.801574 101.66) (end 187.368429 101.66) (width 0.2) (layer "B.Cu") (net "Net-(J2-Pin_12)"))
 (segment (start 201.77 87.258426) (end 201.77 83.35) (width 0.2) (layer "B.Cu") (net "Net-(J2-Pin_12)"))
 (segment (start 171.23 94.18) (end 169.23 96.18) (width 0.2) (layer "B.Cu") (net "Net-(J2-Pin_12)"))
 (segment (start 179.55 95.45) (end 192.38 82.62) (width 0.2) (layer "F.Cu") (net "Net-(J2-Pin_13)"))
 (segment (start 192.38 82.62) (end 198.5 82.62) (width 0.2) (layer "F.Cu") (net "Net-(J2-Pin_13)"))
 (segment (start 172.5 95.45) (end 179.55 95.45) (width 0.2) (layer "F.Cu") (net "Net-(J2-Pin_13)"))
 (segment (start 169.63 97.05) (end 169.63 99.922743) (width 0.2) (layer "B.Cu") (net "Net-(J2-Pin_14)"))
 (segment (start 171.23 95.45) (end 169.63 97.05) (width 0.2) (layer "B.Cu") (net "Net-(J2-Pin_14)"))
 (segment (start 201.37 87.092741) (end 201.37 84.22) (width 0.2) (layer "B.Cu") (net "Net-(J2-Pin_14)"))
 (segment (start 170.967259 101.26) (end 187.202743 101.26) (width 0.2) (layer "B.Cu") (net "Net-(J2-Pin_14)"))
 (segment (start 201.37 84.22) (end 199.77 82.62) (width 0.2) (layer "B.Cu") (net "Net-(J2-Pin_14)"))
 (segment (start 187.202743 101.26) (end 201.37 87.092741) (width 0.2) (layer "B.Cu") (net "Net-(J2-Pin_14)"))
 (segment (start 169.63 99.922743) (end 170.967259 101.26) (width 0.2) (layer "B.Cu") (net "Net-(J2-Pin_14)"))
 (segment (start 172.5 96.72) (end 179.38 96.72) (width 0.2) (layer "F.Cu") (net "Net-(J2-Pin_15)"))
 (segment (start 179.38 96.72) (end 192.21 83.89) (width 0.2) (layer "F.Cu") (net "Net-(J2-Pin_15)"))
 (segment (start 192.21 83.89) (end 198.5 83.89) (width 0.2) (layer "F.Cu") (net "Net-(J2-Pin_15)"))
 (segment (start 187.037057 100.86) (end 200.97 86.927056) (width 0.2) (layer "B.Cu") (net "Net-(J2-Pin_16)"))
 (segment (start 170.03 97.92) (end 170.03 99.757057) (width 0.2) (layer "B.Cu") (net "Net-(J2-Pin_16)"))
 (segment (start 200.97 85.09) (end 199.77 83.89) (width 0.2) (layer "B.Cu") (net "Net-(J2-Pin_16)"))
 (segment (start 171.23 96.72) (end 170.03 97.92) (width 0.2) (layer "B.Cu") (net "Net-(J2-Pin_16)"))
 (segment (start 171.132944 100.86) (end 187.037057 100.86) (width 0.2) (layer "B.Cu") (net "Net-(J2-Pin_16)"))
 (segment (start 170.03 99.757057) (end 171.132944 100.86) (width 0.2) (layer "B.Cu") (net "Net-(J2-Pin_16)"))
 (segment (start 200.97 86.927056) (end 200.97 85.09) (width 0.2) (layer "B.Cu") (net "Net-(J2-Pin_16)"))
 (segment (start 198.5 85.16) (end 192.33 85.16) (width 0.2) (layer "F.Cu") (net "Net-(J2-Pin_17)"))
 (segment (start 172.5 97.99) (end 179.5 97.99) (width 0.2) (layer "F.Cu") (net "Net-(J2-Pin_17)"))
 (segment (start 179.5 97.99) (end 179.51 97.99) (width 0.2) (layer "F.Cu") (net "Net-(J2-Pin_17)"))
 (segment (start 192.33 85.16) (end 179.5 97.99) (width 0.2) (layer "F.Cu") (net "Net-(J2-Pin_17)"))
 (segment (start 200.57 85.96) (end 199.77 85.16) (width 0.2) (layer "B.Cu") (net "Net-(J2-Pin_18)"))
 (segment (start 171.298629 100.46) (end 186.871371 100.46) (width 0.2) (layer "B.Cu") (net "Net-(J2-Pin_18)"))
 (segment (start 170.43 98.79) (end 170.43 99.591371) (width 0.2) (layer "B.Cu") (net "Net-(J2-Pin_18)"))
 (segment (start 171.23 97.99) (end 170.43 98.79) (width 0.2) (layer "B.Cu") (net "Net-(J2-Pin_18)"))
 (segment (start 200.57 86.761371) (end 200.57 85.96) (width 0.2) (layer "B.Cu") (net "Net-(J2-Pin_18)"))
 (segment (start 186.871371 100.46) (end 200.57 86.761371) (width 0.2) (layer "B.Cu") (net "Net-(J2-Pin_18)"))
 (segment (start 170.43 99.591371) (end 171.298629 100.46) (width 0.2) (layer "B.Cu") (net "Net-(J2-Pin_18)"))
 (segment (start 172.5 99.26) (end 179.74 99.26) (width 0.2) (layer "F.Cu") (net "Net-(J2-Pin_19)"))
 (segment (start 179.74 99.26) (end 192.57 86.43) (width 0.2) (layer "F.Cu") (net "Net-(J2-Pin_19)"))
 (segment (start 192.57 86.43) (end 198.5 86.43) (width 0.2) (layer "F.Cu") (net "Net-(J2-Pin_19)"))
 (segment (start 186.14 100.06) (end 199.77 86.43) (width 0.2) (layer "B.Cu") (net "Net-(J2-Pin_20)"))
 (segment (start 172.03 100.06) (end 186.14 100.06) (width 0.2) (layer "B.Cu") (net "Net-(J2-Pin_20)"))
 (segment (start 171.23 99.26) (end 172.03 100.06) (width 0.2) (layer "B.Cu") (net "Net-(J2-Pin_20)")))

